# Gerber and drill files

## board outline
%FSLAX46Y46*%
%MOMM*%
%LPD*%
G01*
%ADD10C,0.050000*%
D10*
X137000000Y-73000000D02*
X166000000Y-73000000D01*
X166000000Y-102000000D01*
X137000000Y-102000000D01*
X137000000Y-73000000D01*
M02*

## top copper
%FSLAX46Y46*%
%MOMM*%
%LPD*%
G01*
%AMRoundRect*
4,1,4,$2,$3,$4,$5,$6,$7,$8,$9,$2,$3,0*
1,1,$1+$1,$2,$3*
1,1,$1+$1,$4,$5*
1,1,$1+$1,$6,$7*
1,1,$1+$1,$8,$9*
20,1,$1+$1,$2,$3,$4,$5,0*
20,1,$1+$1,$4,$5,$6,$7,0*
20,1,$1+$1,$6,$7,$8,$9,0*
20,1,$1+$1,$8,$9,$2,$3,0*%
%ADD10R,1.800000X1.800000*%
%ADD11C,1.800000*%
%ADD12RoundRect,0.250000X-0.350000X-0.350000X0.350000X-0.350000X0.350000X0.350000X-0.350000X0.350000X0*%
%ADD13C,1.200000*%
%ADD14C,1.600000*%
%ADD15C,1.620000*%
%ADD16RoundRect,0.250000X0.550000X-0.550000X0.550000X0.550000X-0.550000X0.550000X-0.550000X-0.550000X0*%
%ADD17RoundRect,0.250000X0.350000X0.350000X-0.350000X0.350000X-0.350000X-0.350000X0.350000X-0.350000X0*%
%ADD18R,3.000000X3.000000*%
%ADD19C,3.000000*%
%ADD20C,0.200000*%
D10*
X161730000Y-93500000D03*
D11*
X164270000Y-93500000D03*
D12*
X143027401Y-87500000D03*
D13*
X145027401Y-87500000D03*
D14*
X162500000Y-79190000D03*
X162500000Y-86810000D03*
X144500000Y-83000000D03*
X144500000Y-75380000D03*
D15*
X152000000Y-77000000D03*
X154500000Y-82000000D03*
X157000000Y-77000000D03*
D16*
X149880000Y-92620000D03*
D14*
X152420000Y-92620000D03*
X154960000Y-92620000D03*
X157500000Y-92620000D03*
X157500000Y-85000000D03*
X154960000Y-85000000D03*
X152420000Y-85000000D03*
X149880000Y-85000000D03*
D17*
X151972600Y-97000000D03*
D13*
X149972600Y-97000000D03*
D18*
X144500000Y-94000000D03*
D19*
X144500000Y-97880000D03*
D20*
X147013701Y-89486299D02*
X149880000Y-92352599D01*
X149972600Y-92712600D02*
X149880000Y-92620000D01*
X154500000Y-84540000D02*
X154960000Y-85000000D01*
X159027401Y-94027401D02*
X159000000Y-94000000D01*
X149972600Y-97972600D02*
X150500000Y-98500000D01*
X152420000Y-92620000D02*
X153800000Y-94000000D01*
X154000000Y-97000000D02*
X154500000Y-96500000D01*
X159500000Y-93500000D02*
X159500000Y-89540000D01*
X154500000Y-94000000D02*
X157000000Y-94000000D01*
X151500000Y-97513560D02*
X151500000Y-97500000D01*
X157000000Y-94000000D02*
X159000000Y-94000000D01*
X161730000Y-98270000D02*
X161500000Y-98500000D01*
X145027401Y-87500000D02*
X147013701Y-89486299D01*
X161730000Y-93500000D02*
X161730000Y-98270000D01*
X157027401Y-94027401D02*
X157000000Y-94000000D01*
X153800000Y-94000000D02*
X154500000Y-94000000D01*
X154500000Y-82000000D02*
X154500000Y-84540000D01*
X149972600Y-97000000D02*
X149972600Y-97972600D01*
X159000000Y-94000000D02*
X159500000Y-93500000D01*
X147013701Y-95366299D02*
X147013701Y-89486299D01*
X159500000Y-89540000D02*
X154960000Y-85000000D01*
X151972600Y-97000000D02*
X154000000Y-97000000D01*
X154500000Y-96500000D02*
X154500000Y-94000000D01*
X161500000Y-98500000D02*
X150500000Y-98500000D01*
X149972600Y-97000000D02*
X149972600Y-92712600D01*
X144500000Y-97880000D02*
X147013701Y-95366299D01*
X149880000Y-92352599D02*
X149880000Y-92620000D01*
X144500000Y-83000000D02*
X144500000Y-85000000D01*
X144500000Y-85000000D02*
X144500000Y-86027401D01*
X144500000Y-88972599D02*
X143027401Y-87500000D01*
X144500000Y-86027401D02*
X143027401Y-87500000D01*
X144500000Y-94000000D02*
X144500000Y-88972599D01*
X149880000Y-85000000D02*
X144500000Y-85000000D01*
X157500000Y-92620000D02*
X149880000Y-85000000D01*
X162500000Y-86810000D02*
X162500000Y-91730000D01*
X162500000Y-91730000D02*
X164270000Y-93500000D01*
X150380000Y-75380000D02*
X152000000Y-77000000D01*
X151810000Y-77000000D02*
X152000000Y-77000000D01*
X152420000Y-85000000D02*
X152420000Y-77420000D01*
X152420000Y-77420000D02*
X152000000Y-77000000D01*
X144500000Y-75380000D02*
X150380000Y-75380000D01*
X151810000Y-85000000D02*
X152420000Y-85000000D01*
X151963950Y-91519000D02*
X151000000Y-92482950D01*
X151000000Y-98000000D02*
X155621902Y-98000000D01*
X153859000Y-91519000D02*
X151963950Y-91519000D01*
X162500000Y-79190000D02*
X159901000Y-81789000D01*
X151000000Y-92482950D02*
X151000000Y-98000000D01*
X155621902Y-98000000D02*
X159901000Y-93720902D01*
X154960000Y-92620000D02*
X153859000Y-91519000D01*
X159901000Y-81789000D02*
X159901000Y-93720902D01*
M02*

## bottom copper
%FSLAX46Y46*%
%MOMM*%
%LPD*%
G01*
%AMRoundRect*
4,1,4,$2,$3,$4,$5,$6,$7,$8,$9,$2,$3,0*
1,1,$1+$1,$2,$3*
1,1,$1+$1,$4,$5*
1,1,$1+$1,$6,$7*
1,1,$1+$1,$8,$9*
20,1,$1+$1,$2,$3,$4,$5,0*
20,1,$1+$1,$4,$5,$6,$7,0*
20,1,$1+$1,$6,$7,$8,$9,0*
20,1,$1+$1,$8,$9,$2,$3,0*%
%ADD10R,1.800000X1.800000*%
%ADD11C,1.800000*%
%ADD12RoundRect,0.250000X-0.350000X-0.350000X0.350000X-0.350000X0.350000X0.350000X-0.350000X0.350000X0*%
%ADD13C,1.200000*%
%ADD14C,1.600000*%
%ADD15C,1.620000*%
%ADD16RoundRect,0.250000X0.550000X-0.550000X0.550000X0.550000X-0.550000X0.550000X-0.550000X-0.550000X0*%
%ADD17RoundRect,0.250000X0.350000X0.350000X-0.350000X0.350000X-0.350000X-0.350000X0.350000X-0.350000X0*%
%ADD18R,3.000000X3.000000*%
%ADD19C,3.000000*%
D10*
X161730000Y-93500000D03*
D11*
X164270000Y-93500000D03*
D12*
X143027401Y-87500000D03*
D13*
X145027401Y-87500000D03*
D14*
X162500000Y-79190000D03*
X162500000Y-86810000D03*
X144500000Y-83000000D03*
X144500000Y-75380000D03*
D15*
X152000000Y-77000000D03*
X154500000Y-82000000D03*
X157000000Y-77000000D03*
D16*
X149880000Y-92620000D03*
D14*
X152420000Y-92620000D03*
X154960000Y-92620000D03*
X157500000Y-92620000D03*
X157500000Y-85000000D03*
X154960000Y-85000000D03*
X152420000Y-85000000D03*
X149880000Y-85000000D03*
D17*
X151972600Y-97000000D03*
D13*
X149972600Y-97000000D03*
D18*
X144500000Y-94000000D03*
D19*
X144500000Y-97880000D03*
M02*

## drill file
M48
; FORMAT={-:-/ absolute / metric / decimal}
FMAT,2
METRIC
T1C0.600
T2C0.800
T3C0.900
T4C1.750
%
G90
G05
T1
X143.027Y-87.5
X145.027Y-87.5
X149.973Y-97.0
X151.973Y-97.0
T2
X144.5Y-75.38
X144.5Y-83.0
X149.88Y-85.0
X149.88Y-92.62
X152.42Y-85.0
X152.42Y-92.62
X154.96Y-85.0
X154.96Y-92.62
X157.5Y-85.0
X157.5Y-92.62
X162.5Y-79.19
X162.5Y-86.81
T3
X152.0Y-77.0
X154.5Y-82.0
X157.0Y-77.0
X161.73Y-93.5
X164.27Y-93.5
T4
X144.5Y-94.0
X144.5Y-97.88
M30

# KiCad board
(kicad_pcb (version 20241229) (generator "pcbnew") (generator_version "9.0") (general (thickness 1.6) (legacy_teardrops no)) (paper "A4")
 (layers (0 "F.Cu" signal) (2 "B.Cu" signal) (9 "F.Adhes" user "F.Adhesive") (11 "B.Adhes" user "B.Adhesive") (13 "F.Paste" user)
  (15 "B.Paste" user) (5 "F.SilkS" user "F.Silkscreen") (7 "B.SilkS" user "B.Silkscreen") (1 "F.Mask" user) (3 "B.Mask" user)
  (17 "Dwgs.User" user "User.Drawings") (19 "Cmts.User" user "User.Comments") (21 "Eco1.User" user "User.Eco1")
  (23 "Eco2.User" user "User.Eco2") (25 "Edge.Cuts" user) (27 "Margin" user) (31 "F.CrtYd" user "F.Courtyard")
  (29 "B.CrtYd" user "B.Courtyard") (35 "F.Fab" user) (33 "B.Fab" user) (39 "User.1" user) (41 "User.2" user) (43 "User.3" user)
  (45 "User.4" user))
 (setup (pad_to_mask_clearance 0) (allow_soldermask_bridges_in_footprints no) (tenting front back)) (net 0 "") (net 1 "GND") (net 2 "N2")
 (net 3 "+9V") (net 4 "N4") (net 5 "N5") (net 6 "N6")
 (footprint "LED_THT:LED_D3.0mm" (layer "F.Cu") (at 161.73 93.5)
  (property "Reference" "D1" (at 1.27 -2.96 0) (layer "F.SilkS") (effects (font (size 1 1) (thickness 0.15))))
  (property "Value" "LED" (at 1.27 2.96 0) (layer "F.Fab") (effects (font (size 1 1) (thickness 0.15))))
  (pad "1" thru_hole rect (at 0 0) (size 1.8 1.8) (drill 0.9) (layers "*.Cu" "*.Mask") (remove_unused_layers no) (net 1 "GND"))
  (pad "2" thru_hole circle (at 2.54 0) (size 1.8 1.8) (drill 0.9) (layers "*.Cu" "*.Mask") (remove_unused_layers no) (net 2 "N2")))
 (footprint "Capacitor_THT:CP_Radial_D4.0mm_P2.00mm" (layer "F.Cu") (at 143.027401 87.5)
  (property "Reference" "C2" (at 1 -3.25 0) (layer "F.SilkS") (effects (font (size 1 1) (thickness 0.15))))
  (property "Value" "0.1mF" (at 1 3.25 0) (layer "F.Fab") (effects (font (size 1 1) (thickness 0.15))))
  (pad "1" thru_hole roundrect (at 0 0) (size 1.2 1.2) (drill 0.6) (layers "*.Cu" "*.Mask") (remove_unused_layers no)
   (roundrect_rratio 0.208333) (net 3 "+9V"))
  (pad "2" thru_hole circle (at 2 0) (size 1.2 1.2) (drill 0.6) (layers "*.Cu" "*.Mask") (remove_unused_layers no) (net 1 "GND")))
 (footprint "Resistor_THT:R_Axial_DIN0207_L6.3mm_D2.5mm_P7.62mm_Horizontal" (layer "F.Cu") (at 162.5 79.19 -90)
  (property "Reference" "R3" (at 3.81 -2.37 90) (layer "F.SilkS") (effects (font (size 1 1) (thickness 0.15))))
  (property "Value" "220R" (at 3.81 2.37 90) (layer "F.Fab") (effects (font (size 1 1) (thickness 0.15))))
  (pad "1" thru_hole circle (at 0 0 270) (size 1.6 1.6) (drill 0.8) (layers "*.Cu" "*.Mask") (remove_unused_layers no) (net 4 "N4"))
  (pad "2" thru_hole circle (at 7.62 0 270) (size 1.6 1.6) (drill 0.8) (layers "*.Cu" "*.Mask") (remove_unused_layers no) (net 2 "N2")))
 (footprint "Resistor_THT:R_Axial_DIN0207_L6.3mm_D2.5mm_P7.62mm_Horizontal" (layer "F.Cu") (at 144.5 83 90)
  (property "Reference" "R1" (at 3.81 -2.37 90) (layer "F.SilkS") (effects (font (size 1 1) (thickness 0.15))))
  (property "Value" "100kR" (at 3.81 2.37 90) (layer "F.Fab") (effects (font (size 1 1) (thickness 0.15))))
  (pad "1" thru_hole circle (at 0 0 90) (size 1.6 1.6) (drill 0.8) (layers "*.Cu" "*.Mask") (remove_unused_layers no) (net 3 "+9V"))
  (pad "2" thru_hole circle (at 7.62 0 90) (size 1.6 1.6) (drill 0.8) (layers "*.Cu" "*.Mask") (remove_unused_layers no) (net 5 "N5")))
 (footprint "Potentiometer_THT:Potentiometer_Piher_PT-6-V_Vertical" (layer "F.Cu") (at 152 77 -90)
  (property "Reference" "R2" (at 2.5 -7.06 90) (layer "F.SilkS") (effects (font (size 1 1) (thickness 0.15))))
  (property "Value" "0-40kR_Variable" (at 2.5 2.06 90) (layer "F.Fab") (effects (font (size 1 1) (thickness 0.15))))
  (pad "1" thru_hole circle (at 0 0 270) (size 1.62 1.62) (drill 0.9) (layers "*.Cu" "*.Mask") (remove_unused_layers no) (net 5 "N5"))
  (pad "2" thru_hole circle (at 5 -2.5 270) (size 1.62 1.62) (drill 0.9) (layers "*.Cu" "*.Mask") (remove_unused_layers no) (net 1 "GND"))
  (pad "3" thru_hole circle (at 0 -5 270) (size 1.62 1.62) (drill 0.9) (layers "*.Cu" "*.Mask") (remove_unused_layers no)))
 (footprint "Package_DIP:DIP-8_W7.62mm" (layer "F.Cu") (at 149.88 92.62 90)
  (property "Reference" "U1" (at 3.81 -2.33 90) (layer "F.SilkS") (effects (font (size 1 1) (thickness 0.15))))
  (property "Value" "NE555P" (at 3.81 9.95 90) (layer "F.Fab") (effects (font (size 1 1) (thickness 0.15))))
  (pad "1" thru_hole roundrect (at 0 0 90) (size 1.6 1.6) (drill 0.8) (layers "*.Cu" "*.Mask") (remove_unused_layers no)
   (roundrect_rratio 0.15625) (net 1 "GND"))
  (pad "2" thru_hole circle (at 0 2.54 90) (size 1.6 1.6) (drill 0.8) (layers "*.Cu" "*.Mask") (remove_unused_layers no) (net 1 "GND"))
  (pad "3" thru_hole circle (at 0 5.08 90) (size 1.6 1.6) (drill 0.8) (layers "*.Cu" "*.Mask") (remove_unused_layers no) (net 4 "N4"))
  (pad "4" thru_hole circle (at 0 7.62 90) (size 1.6 1.6) (drill 0.8) (layers "*.Cu" "*.Mask") (remove_unused_layers no) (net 3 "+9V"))
  (pad "5" thru_hole circle (at 7.62 7.62 90) (size 1.6 1.6) (drill 0.8) (layers "*.Cu" "*.Mask") (remove_unused_layers no) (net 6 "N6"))
  (pad "6" thru_hole circle (at 7.62 5.08 90) (size 1.6 1.6) (drill 0.8) (layers "*.Cu" "*.Mask") (remove_unused_layers no) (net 1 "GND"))
  (pad "7" thru_hole circle (at 7.62 2.54 90) (size 1.6 1.6) (drill 0.8) (layers "*.Cu" "*.Mask") (remove_unused_layers no) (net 5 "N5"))
  (pad "8" thru_hole circle (at 7.62 0 90) (size 1.6 1.6) (drill 0.8) (layers "*.Cu" "*.Mask") (remove_unused_layers no) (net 3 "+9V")))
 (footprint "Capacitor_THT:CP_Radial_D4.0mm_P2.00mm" (layer "F.Cu") (at 151.9726 97 180)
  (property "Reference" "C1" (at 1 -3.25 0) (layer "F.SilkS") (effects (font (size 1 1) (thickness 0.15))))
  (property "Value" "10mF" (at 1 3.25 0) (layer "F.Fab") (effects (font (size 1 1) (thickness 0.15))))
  (pad "1" thru_hole roundrect (at 0 0 180) (size 1.2 1.2) (drill 0.6) (layers "*.Cu" "*.Mask") (remove_unused_layers no)
   (roundrect_rratio 0.208333) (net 1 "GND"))
  (pad "2" thru_hole circle (at 2 0 180) (size 1.2 1.2) (drill 0.6) (layers "*.Cu" "*.Mask") (remove_unused_layers no) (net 1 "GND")))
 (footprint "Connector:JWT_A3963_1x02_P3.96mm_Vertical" (layer "F.Cu") (at 144.5 94 -90)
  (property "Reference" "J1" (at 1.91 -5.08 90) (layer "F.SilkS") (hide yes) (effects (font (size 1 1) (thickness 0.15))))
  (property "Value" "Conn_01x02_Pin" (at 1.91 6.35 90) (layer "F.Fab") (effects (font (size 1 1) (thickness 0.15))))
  (pad "1" thru_hole rect (at 0 0 270) (size 3 3) (drill 1.75) (layers "*.Cu" "*.Mask") (remove_unused_layers no) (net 3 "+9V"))
  (pad "2" thru_hole circle (at 3.88 0 270) (size 3 3) (drill 1.75) (layers "*.Cu" "*.Mask") (remove_unused_layers no) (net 1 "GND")))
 (gr_rect (start 137 73) (end 166 102) (stroke (width 0.05) (type solid)) (fill no) (layer "Edge.Cuts"))
 (segment (start 147.013701 89.486299) (end 149.88 92.352599) (width 0.2) (layer "F.Cu") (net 1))
 (segment (start 149.9726 92.7126) (end 149.88 92.62) (width 0.2) (layer "F.Cu") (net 1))
 (segment (start 154.5 84.54) (end 154.96 85) (width 0.2) (layer "F.Cu") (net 1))
 (segment (start 159.027401 94.027401) (end 159 94) (width 0.2) (layer "F.Cu") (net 1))
 (segment (start 149.9726 97.9726) (end 150.5 98.5) (width 0.2) (layer "F.Cu") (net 1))
 (segment (start 152.42 92.62) (end 153.8 94) (width 0.2) (layer "F.Cu") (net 1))
 (segment (start 154 97) (end 154.5 96.5) (width 0.2) (layer "F.Cu") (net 1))
 (segment (start 159.5 93.5) (end 159.5 89.54) (width 0.2) (layer "F.Cu") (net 1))
 (segment (start 154.5 94) (end 157 94) (width 0.2) (layer "F.Cu") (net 1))
 (segment (start 151.5 97.51356) (end 151.5 97.5) (width 0.2) (layer "F.Cu") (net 1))
 (segment (start 157 94) (end 159 94) (width 0.2) (layer "F.Cu") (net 1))
 (segment (start 161.73 98.27) (end 161.5 98.5) (width 0.2) (layer "F.Cu") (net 1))
 (segment (start 145.027401 87.5) (end 147.013701 89.486299) (width 0.2) (layer "F.Cu") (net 1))
 (segment (start 161.73 93.5) (end 161.73 98.27) (width 0.2) (layer "F.Cu") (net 1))
 (segment (start 157.027401 94.027401) (end 157 94) (width 0.2) (layer "F.Cu") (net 1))
 (segment (start 153.8 94) (end 154.5 94) (width 0.2) (layer "F.Cu") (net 1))
 (segment (start 154.5 82) (end 154.5 84.54) (width 0.2) (layer "F.Cu") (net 1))
 (segment (start 149.9726 97) (end 149.9726 97.9726) (width 0.2) (layer "F.Cu") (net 1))
 (segment (start 159 94) (end 159.5 93.5) (width 0.2) (layer "F.Cu") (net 1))
 (segment (start 147.013701 95.366299) (end 147.013701 89.486299) (width 0.2) (layer "F.Cu") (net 1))
 (segment (start 159.5 89.54) (end 154.96 85) (width 0.2) (layer "F.Cu") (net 1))
 (segment (start 151.9726 97) (end 154 97) (width 0.2) (layer "F.Cu") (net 1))
 (segment (start 154.5 96.5) (end 154.5 94) (width 0.2) (layer "F.Cu") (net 1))
 (segment (start 161.5 98.5) (end 150.5 98.5) (width 0.2) (layer "F.Cu") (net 1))
 (segment (start 149.9726 97) (end 149.9726 92.7126) (width 0.2) (layer "F.Cu") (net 1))
 (segment (start 144.5 97.88) (end 147.013701 95.366299) (width 0.2) (layer "F.Cu") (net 1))
 (segment (start 149.88 92.352599) (end 149.88 92.62) (width 0.2) (layer "F.Cu") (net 1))
 (segment (start 144.5 83) (end 144.5 85) (width 0.2) (layer "F.Cu") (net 3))
 (segment (start 144.5 85) (end 144.5 86.027401) (width 0.2) (layer "F.Cu") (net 3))
 (segment (start 144.5 88.972599) (end 143.027401 87.5) (width 0.2) (layer "F.Cu") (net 3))
 (segment (start 144.5 86.027401) (end 143.027401 87.5) (width 0.2) (layer "F.Cu") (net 3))
 (segment (start 144.5 94) (end 144.5 88.972599) (width 0.2) (layer "F.Cu") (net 3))
 (segment (start 149.88 85) (end 144.5 85) (width 0.2) (layer "F.Cu") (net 3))
 (segment (start 157.5 92.62) (end 149.88 85) (width 0.2) (layer "F.Cu") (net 3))
 (segment (start 162.5 86.81) (end 162.5 91.73) (width 0.2) (layer "F.Cu") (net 2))
 (segment (start 162.5 91.73) (end 164.27 93.5) (width 0.2) (layer "F.Cu") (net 2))
 (segment (start 150.38 75.38) (end 152 77) (width 0.2) (layer "F.Cu") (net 5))
 (segment (start 151.81 77) (end 152 77) (width 0.2) (layer "F.Cu") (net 5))
 (segment (start 152.42 85) (end 152.42 77.42) (width 0.2) (layer "F.Cu") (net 5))
 (segment (start 152.42 77.42) (end 152 77) (width 0.2) (layer "F.Cu") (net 5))
 (segment (start 144.5 75.38) (end 150.38 75.38) (width 0.2) (layer "F.Cu") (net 5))
 (segment (start 151.81 85) (end 152.42 85) (width 0.2) (layer "F.Cu") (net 5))
 (segment (start 151.96395 91.519) (end 151 92.48295) (width 0.2) (layer "F.Cu") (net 4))
 (segment (start 151 98) (end 155.621902 98) (width 0.2) (layer "F.Cu") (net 4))
 (segment (start 153.859 91.519) (end 151.96395 91.519) (width 0.2) (layer "F.Cu") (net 4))
 (segment (start 162.5 79.19) (end 159.901 81.789) (width 0.2) (layer "F.Cu") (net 4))
 (segment (start 151 92.48295) (end 151 98) (width 0.2) (layer "F.Cu") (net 4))
 (segment (start 155.621902 98) (end 159.901 93.720902) (width 0.2) (layer "F.Cu") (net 4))
 (segment (start 154.96 92.62) (end 153.859 91.519) (width 0.2) (layer "F.Cu") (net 4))
 (segment (start 159.901 81.789) (end 159.901 93.720902) (width 0.2) (layer "F.Cu") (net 4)))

